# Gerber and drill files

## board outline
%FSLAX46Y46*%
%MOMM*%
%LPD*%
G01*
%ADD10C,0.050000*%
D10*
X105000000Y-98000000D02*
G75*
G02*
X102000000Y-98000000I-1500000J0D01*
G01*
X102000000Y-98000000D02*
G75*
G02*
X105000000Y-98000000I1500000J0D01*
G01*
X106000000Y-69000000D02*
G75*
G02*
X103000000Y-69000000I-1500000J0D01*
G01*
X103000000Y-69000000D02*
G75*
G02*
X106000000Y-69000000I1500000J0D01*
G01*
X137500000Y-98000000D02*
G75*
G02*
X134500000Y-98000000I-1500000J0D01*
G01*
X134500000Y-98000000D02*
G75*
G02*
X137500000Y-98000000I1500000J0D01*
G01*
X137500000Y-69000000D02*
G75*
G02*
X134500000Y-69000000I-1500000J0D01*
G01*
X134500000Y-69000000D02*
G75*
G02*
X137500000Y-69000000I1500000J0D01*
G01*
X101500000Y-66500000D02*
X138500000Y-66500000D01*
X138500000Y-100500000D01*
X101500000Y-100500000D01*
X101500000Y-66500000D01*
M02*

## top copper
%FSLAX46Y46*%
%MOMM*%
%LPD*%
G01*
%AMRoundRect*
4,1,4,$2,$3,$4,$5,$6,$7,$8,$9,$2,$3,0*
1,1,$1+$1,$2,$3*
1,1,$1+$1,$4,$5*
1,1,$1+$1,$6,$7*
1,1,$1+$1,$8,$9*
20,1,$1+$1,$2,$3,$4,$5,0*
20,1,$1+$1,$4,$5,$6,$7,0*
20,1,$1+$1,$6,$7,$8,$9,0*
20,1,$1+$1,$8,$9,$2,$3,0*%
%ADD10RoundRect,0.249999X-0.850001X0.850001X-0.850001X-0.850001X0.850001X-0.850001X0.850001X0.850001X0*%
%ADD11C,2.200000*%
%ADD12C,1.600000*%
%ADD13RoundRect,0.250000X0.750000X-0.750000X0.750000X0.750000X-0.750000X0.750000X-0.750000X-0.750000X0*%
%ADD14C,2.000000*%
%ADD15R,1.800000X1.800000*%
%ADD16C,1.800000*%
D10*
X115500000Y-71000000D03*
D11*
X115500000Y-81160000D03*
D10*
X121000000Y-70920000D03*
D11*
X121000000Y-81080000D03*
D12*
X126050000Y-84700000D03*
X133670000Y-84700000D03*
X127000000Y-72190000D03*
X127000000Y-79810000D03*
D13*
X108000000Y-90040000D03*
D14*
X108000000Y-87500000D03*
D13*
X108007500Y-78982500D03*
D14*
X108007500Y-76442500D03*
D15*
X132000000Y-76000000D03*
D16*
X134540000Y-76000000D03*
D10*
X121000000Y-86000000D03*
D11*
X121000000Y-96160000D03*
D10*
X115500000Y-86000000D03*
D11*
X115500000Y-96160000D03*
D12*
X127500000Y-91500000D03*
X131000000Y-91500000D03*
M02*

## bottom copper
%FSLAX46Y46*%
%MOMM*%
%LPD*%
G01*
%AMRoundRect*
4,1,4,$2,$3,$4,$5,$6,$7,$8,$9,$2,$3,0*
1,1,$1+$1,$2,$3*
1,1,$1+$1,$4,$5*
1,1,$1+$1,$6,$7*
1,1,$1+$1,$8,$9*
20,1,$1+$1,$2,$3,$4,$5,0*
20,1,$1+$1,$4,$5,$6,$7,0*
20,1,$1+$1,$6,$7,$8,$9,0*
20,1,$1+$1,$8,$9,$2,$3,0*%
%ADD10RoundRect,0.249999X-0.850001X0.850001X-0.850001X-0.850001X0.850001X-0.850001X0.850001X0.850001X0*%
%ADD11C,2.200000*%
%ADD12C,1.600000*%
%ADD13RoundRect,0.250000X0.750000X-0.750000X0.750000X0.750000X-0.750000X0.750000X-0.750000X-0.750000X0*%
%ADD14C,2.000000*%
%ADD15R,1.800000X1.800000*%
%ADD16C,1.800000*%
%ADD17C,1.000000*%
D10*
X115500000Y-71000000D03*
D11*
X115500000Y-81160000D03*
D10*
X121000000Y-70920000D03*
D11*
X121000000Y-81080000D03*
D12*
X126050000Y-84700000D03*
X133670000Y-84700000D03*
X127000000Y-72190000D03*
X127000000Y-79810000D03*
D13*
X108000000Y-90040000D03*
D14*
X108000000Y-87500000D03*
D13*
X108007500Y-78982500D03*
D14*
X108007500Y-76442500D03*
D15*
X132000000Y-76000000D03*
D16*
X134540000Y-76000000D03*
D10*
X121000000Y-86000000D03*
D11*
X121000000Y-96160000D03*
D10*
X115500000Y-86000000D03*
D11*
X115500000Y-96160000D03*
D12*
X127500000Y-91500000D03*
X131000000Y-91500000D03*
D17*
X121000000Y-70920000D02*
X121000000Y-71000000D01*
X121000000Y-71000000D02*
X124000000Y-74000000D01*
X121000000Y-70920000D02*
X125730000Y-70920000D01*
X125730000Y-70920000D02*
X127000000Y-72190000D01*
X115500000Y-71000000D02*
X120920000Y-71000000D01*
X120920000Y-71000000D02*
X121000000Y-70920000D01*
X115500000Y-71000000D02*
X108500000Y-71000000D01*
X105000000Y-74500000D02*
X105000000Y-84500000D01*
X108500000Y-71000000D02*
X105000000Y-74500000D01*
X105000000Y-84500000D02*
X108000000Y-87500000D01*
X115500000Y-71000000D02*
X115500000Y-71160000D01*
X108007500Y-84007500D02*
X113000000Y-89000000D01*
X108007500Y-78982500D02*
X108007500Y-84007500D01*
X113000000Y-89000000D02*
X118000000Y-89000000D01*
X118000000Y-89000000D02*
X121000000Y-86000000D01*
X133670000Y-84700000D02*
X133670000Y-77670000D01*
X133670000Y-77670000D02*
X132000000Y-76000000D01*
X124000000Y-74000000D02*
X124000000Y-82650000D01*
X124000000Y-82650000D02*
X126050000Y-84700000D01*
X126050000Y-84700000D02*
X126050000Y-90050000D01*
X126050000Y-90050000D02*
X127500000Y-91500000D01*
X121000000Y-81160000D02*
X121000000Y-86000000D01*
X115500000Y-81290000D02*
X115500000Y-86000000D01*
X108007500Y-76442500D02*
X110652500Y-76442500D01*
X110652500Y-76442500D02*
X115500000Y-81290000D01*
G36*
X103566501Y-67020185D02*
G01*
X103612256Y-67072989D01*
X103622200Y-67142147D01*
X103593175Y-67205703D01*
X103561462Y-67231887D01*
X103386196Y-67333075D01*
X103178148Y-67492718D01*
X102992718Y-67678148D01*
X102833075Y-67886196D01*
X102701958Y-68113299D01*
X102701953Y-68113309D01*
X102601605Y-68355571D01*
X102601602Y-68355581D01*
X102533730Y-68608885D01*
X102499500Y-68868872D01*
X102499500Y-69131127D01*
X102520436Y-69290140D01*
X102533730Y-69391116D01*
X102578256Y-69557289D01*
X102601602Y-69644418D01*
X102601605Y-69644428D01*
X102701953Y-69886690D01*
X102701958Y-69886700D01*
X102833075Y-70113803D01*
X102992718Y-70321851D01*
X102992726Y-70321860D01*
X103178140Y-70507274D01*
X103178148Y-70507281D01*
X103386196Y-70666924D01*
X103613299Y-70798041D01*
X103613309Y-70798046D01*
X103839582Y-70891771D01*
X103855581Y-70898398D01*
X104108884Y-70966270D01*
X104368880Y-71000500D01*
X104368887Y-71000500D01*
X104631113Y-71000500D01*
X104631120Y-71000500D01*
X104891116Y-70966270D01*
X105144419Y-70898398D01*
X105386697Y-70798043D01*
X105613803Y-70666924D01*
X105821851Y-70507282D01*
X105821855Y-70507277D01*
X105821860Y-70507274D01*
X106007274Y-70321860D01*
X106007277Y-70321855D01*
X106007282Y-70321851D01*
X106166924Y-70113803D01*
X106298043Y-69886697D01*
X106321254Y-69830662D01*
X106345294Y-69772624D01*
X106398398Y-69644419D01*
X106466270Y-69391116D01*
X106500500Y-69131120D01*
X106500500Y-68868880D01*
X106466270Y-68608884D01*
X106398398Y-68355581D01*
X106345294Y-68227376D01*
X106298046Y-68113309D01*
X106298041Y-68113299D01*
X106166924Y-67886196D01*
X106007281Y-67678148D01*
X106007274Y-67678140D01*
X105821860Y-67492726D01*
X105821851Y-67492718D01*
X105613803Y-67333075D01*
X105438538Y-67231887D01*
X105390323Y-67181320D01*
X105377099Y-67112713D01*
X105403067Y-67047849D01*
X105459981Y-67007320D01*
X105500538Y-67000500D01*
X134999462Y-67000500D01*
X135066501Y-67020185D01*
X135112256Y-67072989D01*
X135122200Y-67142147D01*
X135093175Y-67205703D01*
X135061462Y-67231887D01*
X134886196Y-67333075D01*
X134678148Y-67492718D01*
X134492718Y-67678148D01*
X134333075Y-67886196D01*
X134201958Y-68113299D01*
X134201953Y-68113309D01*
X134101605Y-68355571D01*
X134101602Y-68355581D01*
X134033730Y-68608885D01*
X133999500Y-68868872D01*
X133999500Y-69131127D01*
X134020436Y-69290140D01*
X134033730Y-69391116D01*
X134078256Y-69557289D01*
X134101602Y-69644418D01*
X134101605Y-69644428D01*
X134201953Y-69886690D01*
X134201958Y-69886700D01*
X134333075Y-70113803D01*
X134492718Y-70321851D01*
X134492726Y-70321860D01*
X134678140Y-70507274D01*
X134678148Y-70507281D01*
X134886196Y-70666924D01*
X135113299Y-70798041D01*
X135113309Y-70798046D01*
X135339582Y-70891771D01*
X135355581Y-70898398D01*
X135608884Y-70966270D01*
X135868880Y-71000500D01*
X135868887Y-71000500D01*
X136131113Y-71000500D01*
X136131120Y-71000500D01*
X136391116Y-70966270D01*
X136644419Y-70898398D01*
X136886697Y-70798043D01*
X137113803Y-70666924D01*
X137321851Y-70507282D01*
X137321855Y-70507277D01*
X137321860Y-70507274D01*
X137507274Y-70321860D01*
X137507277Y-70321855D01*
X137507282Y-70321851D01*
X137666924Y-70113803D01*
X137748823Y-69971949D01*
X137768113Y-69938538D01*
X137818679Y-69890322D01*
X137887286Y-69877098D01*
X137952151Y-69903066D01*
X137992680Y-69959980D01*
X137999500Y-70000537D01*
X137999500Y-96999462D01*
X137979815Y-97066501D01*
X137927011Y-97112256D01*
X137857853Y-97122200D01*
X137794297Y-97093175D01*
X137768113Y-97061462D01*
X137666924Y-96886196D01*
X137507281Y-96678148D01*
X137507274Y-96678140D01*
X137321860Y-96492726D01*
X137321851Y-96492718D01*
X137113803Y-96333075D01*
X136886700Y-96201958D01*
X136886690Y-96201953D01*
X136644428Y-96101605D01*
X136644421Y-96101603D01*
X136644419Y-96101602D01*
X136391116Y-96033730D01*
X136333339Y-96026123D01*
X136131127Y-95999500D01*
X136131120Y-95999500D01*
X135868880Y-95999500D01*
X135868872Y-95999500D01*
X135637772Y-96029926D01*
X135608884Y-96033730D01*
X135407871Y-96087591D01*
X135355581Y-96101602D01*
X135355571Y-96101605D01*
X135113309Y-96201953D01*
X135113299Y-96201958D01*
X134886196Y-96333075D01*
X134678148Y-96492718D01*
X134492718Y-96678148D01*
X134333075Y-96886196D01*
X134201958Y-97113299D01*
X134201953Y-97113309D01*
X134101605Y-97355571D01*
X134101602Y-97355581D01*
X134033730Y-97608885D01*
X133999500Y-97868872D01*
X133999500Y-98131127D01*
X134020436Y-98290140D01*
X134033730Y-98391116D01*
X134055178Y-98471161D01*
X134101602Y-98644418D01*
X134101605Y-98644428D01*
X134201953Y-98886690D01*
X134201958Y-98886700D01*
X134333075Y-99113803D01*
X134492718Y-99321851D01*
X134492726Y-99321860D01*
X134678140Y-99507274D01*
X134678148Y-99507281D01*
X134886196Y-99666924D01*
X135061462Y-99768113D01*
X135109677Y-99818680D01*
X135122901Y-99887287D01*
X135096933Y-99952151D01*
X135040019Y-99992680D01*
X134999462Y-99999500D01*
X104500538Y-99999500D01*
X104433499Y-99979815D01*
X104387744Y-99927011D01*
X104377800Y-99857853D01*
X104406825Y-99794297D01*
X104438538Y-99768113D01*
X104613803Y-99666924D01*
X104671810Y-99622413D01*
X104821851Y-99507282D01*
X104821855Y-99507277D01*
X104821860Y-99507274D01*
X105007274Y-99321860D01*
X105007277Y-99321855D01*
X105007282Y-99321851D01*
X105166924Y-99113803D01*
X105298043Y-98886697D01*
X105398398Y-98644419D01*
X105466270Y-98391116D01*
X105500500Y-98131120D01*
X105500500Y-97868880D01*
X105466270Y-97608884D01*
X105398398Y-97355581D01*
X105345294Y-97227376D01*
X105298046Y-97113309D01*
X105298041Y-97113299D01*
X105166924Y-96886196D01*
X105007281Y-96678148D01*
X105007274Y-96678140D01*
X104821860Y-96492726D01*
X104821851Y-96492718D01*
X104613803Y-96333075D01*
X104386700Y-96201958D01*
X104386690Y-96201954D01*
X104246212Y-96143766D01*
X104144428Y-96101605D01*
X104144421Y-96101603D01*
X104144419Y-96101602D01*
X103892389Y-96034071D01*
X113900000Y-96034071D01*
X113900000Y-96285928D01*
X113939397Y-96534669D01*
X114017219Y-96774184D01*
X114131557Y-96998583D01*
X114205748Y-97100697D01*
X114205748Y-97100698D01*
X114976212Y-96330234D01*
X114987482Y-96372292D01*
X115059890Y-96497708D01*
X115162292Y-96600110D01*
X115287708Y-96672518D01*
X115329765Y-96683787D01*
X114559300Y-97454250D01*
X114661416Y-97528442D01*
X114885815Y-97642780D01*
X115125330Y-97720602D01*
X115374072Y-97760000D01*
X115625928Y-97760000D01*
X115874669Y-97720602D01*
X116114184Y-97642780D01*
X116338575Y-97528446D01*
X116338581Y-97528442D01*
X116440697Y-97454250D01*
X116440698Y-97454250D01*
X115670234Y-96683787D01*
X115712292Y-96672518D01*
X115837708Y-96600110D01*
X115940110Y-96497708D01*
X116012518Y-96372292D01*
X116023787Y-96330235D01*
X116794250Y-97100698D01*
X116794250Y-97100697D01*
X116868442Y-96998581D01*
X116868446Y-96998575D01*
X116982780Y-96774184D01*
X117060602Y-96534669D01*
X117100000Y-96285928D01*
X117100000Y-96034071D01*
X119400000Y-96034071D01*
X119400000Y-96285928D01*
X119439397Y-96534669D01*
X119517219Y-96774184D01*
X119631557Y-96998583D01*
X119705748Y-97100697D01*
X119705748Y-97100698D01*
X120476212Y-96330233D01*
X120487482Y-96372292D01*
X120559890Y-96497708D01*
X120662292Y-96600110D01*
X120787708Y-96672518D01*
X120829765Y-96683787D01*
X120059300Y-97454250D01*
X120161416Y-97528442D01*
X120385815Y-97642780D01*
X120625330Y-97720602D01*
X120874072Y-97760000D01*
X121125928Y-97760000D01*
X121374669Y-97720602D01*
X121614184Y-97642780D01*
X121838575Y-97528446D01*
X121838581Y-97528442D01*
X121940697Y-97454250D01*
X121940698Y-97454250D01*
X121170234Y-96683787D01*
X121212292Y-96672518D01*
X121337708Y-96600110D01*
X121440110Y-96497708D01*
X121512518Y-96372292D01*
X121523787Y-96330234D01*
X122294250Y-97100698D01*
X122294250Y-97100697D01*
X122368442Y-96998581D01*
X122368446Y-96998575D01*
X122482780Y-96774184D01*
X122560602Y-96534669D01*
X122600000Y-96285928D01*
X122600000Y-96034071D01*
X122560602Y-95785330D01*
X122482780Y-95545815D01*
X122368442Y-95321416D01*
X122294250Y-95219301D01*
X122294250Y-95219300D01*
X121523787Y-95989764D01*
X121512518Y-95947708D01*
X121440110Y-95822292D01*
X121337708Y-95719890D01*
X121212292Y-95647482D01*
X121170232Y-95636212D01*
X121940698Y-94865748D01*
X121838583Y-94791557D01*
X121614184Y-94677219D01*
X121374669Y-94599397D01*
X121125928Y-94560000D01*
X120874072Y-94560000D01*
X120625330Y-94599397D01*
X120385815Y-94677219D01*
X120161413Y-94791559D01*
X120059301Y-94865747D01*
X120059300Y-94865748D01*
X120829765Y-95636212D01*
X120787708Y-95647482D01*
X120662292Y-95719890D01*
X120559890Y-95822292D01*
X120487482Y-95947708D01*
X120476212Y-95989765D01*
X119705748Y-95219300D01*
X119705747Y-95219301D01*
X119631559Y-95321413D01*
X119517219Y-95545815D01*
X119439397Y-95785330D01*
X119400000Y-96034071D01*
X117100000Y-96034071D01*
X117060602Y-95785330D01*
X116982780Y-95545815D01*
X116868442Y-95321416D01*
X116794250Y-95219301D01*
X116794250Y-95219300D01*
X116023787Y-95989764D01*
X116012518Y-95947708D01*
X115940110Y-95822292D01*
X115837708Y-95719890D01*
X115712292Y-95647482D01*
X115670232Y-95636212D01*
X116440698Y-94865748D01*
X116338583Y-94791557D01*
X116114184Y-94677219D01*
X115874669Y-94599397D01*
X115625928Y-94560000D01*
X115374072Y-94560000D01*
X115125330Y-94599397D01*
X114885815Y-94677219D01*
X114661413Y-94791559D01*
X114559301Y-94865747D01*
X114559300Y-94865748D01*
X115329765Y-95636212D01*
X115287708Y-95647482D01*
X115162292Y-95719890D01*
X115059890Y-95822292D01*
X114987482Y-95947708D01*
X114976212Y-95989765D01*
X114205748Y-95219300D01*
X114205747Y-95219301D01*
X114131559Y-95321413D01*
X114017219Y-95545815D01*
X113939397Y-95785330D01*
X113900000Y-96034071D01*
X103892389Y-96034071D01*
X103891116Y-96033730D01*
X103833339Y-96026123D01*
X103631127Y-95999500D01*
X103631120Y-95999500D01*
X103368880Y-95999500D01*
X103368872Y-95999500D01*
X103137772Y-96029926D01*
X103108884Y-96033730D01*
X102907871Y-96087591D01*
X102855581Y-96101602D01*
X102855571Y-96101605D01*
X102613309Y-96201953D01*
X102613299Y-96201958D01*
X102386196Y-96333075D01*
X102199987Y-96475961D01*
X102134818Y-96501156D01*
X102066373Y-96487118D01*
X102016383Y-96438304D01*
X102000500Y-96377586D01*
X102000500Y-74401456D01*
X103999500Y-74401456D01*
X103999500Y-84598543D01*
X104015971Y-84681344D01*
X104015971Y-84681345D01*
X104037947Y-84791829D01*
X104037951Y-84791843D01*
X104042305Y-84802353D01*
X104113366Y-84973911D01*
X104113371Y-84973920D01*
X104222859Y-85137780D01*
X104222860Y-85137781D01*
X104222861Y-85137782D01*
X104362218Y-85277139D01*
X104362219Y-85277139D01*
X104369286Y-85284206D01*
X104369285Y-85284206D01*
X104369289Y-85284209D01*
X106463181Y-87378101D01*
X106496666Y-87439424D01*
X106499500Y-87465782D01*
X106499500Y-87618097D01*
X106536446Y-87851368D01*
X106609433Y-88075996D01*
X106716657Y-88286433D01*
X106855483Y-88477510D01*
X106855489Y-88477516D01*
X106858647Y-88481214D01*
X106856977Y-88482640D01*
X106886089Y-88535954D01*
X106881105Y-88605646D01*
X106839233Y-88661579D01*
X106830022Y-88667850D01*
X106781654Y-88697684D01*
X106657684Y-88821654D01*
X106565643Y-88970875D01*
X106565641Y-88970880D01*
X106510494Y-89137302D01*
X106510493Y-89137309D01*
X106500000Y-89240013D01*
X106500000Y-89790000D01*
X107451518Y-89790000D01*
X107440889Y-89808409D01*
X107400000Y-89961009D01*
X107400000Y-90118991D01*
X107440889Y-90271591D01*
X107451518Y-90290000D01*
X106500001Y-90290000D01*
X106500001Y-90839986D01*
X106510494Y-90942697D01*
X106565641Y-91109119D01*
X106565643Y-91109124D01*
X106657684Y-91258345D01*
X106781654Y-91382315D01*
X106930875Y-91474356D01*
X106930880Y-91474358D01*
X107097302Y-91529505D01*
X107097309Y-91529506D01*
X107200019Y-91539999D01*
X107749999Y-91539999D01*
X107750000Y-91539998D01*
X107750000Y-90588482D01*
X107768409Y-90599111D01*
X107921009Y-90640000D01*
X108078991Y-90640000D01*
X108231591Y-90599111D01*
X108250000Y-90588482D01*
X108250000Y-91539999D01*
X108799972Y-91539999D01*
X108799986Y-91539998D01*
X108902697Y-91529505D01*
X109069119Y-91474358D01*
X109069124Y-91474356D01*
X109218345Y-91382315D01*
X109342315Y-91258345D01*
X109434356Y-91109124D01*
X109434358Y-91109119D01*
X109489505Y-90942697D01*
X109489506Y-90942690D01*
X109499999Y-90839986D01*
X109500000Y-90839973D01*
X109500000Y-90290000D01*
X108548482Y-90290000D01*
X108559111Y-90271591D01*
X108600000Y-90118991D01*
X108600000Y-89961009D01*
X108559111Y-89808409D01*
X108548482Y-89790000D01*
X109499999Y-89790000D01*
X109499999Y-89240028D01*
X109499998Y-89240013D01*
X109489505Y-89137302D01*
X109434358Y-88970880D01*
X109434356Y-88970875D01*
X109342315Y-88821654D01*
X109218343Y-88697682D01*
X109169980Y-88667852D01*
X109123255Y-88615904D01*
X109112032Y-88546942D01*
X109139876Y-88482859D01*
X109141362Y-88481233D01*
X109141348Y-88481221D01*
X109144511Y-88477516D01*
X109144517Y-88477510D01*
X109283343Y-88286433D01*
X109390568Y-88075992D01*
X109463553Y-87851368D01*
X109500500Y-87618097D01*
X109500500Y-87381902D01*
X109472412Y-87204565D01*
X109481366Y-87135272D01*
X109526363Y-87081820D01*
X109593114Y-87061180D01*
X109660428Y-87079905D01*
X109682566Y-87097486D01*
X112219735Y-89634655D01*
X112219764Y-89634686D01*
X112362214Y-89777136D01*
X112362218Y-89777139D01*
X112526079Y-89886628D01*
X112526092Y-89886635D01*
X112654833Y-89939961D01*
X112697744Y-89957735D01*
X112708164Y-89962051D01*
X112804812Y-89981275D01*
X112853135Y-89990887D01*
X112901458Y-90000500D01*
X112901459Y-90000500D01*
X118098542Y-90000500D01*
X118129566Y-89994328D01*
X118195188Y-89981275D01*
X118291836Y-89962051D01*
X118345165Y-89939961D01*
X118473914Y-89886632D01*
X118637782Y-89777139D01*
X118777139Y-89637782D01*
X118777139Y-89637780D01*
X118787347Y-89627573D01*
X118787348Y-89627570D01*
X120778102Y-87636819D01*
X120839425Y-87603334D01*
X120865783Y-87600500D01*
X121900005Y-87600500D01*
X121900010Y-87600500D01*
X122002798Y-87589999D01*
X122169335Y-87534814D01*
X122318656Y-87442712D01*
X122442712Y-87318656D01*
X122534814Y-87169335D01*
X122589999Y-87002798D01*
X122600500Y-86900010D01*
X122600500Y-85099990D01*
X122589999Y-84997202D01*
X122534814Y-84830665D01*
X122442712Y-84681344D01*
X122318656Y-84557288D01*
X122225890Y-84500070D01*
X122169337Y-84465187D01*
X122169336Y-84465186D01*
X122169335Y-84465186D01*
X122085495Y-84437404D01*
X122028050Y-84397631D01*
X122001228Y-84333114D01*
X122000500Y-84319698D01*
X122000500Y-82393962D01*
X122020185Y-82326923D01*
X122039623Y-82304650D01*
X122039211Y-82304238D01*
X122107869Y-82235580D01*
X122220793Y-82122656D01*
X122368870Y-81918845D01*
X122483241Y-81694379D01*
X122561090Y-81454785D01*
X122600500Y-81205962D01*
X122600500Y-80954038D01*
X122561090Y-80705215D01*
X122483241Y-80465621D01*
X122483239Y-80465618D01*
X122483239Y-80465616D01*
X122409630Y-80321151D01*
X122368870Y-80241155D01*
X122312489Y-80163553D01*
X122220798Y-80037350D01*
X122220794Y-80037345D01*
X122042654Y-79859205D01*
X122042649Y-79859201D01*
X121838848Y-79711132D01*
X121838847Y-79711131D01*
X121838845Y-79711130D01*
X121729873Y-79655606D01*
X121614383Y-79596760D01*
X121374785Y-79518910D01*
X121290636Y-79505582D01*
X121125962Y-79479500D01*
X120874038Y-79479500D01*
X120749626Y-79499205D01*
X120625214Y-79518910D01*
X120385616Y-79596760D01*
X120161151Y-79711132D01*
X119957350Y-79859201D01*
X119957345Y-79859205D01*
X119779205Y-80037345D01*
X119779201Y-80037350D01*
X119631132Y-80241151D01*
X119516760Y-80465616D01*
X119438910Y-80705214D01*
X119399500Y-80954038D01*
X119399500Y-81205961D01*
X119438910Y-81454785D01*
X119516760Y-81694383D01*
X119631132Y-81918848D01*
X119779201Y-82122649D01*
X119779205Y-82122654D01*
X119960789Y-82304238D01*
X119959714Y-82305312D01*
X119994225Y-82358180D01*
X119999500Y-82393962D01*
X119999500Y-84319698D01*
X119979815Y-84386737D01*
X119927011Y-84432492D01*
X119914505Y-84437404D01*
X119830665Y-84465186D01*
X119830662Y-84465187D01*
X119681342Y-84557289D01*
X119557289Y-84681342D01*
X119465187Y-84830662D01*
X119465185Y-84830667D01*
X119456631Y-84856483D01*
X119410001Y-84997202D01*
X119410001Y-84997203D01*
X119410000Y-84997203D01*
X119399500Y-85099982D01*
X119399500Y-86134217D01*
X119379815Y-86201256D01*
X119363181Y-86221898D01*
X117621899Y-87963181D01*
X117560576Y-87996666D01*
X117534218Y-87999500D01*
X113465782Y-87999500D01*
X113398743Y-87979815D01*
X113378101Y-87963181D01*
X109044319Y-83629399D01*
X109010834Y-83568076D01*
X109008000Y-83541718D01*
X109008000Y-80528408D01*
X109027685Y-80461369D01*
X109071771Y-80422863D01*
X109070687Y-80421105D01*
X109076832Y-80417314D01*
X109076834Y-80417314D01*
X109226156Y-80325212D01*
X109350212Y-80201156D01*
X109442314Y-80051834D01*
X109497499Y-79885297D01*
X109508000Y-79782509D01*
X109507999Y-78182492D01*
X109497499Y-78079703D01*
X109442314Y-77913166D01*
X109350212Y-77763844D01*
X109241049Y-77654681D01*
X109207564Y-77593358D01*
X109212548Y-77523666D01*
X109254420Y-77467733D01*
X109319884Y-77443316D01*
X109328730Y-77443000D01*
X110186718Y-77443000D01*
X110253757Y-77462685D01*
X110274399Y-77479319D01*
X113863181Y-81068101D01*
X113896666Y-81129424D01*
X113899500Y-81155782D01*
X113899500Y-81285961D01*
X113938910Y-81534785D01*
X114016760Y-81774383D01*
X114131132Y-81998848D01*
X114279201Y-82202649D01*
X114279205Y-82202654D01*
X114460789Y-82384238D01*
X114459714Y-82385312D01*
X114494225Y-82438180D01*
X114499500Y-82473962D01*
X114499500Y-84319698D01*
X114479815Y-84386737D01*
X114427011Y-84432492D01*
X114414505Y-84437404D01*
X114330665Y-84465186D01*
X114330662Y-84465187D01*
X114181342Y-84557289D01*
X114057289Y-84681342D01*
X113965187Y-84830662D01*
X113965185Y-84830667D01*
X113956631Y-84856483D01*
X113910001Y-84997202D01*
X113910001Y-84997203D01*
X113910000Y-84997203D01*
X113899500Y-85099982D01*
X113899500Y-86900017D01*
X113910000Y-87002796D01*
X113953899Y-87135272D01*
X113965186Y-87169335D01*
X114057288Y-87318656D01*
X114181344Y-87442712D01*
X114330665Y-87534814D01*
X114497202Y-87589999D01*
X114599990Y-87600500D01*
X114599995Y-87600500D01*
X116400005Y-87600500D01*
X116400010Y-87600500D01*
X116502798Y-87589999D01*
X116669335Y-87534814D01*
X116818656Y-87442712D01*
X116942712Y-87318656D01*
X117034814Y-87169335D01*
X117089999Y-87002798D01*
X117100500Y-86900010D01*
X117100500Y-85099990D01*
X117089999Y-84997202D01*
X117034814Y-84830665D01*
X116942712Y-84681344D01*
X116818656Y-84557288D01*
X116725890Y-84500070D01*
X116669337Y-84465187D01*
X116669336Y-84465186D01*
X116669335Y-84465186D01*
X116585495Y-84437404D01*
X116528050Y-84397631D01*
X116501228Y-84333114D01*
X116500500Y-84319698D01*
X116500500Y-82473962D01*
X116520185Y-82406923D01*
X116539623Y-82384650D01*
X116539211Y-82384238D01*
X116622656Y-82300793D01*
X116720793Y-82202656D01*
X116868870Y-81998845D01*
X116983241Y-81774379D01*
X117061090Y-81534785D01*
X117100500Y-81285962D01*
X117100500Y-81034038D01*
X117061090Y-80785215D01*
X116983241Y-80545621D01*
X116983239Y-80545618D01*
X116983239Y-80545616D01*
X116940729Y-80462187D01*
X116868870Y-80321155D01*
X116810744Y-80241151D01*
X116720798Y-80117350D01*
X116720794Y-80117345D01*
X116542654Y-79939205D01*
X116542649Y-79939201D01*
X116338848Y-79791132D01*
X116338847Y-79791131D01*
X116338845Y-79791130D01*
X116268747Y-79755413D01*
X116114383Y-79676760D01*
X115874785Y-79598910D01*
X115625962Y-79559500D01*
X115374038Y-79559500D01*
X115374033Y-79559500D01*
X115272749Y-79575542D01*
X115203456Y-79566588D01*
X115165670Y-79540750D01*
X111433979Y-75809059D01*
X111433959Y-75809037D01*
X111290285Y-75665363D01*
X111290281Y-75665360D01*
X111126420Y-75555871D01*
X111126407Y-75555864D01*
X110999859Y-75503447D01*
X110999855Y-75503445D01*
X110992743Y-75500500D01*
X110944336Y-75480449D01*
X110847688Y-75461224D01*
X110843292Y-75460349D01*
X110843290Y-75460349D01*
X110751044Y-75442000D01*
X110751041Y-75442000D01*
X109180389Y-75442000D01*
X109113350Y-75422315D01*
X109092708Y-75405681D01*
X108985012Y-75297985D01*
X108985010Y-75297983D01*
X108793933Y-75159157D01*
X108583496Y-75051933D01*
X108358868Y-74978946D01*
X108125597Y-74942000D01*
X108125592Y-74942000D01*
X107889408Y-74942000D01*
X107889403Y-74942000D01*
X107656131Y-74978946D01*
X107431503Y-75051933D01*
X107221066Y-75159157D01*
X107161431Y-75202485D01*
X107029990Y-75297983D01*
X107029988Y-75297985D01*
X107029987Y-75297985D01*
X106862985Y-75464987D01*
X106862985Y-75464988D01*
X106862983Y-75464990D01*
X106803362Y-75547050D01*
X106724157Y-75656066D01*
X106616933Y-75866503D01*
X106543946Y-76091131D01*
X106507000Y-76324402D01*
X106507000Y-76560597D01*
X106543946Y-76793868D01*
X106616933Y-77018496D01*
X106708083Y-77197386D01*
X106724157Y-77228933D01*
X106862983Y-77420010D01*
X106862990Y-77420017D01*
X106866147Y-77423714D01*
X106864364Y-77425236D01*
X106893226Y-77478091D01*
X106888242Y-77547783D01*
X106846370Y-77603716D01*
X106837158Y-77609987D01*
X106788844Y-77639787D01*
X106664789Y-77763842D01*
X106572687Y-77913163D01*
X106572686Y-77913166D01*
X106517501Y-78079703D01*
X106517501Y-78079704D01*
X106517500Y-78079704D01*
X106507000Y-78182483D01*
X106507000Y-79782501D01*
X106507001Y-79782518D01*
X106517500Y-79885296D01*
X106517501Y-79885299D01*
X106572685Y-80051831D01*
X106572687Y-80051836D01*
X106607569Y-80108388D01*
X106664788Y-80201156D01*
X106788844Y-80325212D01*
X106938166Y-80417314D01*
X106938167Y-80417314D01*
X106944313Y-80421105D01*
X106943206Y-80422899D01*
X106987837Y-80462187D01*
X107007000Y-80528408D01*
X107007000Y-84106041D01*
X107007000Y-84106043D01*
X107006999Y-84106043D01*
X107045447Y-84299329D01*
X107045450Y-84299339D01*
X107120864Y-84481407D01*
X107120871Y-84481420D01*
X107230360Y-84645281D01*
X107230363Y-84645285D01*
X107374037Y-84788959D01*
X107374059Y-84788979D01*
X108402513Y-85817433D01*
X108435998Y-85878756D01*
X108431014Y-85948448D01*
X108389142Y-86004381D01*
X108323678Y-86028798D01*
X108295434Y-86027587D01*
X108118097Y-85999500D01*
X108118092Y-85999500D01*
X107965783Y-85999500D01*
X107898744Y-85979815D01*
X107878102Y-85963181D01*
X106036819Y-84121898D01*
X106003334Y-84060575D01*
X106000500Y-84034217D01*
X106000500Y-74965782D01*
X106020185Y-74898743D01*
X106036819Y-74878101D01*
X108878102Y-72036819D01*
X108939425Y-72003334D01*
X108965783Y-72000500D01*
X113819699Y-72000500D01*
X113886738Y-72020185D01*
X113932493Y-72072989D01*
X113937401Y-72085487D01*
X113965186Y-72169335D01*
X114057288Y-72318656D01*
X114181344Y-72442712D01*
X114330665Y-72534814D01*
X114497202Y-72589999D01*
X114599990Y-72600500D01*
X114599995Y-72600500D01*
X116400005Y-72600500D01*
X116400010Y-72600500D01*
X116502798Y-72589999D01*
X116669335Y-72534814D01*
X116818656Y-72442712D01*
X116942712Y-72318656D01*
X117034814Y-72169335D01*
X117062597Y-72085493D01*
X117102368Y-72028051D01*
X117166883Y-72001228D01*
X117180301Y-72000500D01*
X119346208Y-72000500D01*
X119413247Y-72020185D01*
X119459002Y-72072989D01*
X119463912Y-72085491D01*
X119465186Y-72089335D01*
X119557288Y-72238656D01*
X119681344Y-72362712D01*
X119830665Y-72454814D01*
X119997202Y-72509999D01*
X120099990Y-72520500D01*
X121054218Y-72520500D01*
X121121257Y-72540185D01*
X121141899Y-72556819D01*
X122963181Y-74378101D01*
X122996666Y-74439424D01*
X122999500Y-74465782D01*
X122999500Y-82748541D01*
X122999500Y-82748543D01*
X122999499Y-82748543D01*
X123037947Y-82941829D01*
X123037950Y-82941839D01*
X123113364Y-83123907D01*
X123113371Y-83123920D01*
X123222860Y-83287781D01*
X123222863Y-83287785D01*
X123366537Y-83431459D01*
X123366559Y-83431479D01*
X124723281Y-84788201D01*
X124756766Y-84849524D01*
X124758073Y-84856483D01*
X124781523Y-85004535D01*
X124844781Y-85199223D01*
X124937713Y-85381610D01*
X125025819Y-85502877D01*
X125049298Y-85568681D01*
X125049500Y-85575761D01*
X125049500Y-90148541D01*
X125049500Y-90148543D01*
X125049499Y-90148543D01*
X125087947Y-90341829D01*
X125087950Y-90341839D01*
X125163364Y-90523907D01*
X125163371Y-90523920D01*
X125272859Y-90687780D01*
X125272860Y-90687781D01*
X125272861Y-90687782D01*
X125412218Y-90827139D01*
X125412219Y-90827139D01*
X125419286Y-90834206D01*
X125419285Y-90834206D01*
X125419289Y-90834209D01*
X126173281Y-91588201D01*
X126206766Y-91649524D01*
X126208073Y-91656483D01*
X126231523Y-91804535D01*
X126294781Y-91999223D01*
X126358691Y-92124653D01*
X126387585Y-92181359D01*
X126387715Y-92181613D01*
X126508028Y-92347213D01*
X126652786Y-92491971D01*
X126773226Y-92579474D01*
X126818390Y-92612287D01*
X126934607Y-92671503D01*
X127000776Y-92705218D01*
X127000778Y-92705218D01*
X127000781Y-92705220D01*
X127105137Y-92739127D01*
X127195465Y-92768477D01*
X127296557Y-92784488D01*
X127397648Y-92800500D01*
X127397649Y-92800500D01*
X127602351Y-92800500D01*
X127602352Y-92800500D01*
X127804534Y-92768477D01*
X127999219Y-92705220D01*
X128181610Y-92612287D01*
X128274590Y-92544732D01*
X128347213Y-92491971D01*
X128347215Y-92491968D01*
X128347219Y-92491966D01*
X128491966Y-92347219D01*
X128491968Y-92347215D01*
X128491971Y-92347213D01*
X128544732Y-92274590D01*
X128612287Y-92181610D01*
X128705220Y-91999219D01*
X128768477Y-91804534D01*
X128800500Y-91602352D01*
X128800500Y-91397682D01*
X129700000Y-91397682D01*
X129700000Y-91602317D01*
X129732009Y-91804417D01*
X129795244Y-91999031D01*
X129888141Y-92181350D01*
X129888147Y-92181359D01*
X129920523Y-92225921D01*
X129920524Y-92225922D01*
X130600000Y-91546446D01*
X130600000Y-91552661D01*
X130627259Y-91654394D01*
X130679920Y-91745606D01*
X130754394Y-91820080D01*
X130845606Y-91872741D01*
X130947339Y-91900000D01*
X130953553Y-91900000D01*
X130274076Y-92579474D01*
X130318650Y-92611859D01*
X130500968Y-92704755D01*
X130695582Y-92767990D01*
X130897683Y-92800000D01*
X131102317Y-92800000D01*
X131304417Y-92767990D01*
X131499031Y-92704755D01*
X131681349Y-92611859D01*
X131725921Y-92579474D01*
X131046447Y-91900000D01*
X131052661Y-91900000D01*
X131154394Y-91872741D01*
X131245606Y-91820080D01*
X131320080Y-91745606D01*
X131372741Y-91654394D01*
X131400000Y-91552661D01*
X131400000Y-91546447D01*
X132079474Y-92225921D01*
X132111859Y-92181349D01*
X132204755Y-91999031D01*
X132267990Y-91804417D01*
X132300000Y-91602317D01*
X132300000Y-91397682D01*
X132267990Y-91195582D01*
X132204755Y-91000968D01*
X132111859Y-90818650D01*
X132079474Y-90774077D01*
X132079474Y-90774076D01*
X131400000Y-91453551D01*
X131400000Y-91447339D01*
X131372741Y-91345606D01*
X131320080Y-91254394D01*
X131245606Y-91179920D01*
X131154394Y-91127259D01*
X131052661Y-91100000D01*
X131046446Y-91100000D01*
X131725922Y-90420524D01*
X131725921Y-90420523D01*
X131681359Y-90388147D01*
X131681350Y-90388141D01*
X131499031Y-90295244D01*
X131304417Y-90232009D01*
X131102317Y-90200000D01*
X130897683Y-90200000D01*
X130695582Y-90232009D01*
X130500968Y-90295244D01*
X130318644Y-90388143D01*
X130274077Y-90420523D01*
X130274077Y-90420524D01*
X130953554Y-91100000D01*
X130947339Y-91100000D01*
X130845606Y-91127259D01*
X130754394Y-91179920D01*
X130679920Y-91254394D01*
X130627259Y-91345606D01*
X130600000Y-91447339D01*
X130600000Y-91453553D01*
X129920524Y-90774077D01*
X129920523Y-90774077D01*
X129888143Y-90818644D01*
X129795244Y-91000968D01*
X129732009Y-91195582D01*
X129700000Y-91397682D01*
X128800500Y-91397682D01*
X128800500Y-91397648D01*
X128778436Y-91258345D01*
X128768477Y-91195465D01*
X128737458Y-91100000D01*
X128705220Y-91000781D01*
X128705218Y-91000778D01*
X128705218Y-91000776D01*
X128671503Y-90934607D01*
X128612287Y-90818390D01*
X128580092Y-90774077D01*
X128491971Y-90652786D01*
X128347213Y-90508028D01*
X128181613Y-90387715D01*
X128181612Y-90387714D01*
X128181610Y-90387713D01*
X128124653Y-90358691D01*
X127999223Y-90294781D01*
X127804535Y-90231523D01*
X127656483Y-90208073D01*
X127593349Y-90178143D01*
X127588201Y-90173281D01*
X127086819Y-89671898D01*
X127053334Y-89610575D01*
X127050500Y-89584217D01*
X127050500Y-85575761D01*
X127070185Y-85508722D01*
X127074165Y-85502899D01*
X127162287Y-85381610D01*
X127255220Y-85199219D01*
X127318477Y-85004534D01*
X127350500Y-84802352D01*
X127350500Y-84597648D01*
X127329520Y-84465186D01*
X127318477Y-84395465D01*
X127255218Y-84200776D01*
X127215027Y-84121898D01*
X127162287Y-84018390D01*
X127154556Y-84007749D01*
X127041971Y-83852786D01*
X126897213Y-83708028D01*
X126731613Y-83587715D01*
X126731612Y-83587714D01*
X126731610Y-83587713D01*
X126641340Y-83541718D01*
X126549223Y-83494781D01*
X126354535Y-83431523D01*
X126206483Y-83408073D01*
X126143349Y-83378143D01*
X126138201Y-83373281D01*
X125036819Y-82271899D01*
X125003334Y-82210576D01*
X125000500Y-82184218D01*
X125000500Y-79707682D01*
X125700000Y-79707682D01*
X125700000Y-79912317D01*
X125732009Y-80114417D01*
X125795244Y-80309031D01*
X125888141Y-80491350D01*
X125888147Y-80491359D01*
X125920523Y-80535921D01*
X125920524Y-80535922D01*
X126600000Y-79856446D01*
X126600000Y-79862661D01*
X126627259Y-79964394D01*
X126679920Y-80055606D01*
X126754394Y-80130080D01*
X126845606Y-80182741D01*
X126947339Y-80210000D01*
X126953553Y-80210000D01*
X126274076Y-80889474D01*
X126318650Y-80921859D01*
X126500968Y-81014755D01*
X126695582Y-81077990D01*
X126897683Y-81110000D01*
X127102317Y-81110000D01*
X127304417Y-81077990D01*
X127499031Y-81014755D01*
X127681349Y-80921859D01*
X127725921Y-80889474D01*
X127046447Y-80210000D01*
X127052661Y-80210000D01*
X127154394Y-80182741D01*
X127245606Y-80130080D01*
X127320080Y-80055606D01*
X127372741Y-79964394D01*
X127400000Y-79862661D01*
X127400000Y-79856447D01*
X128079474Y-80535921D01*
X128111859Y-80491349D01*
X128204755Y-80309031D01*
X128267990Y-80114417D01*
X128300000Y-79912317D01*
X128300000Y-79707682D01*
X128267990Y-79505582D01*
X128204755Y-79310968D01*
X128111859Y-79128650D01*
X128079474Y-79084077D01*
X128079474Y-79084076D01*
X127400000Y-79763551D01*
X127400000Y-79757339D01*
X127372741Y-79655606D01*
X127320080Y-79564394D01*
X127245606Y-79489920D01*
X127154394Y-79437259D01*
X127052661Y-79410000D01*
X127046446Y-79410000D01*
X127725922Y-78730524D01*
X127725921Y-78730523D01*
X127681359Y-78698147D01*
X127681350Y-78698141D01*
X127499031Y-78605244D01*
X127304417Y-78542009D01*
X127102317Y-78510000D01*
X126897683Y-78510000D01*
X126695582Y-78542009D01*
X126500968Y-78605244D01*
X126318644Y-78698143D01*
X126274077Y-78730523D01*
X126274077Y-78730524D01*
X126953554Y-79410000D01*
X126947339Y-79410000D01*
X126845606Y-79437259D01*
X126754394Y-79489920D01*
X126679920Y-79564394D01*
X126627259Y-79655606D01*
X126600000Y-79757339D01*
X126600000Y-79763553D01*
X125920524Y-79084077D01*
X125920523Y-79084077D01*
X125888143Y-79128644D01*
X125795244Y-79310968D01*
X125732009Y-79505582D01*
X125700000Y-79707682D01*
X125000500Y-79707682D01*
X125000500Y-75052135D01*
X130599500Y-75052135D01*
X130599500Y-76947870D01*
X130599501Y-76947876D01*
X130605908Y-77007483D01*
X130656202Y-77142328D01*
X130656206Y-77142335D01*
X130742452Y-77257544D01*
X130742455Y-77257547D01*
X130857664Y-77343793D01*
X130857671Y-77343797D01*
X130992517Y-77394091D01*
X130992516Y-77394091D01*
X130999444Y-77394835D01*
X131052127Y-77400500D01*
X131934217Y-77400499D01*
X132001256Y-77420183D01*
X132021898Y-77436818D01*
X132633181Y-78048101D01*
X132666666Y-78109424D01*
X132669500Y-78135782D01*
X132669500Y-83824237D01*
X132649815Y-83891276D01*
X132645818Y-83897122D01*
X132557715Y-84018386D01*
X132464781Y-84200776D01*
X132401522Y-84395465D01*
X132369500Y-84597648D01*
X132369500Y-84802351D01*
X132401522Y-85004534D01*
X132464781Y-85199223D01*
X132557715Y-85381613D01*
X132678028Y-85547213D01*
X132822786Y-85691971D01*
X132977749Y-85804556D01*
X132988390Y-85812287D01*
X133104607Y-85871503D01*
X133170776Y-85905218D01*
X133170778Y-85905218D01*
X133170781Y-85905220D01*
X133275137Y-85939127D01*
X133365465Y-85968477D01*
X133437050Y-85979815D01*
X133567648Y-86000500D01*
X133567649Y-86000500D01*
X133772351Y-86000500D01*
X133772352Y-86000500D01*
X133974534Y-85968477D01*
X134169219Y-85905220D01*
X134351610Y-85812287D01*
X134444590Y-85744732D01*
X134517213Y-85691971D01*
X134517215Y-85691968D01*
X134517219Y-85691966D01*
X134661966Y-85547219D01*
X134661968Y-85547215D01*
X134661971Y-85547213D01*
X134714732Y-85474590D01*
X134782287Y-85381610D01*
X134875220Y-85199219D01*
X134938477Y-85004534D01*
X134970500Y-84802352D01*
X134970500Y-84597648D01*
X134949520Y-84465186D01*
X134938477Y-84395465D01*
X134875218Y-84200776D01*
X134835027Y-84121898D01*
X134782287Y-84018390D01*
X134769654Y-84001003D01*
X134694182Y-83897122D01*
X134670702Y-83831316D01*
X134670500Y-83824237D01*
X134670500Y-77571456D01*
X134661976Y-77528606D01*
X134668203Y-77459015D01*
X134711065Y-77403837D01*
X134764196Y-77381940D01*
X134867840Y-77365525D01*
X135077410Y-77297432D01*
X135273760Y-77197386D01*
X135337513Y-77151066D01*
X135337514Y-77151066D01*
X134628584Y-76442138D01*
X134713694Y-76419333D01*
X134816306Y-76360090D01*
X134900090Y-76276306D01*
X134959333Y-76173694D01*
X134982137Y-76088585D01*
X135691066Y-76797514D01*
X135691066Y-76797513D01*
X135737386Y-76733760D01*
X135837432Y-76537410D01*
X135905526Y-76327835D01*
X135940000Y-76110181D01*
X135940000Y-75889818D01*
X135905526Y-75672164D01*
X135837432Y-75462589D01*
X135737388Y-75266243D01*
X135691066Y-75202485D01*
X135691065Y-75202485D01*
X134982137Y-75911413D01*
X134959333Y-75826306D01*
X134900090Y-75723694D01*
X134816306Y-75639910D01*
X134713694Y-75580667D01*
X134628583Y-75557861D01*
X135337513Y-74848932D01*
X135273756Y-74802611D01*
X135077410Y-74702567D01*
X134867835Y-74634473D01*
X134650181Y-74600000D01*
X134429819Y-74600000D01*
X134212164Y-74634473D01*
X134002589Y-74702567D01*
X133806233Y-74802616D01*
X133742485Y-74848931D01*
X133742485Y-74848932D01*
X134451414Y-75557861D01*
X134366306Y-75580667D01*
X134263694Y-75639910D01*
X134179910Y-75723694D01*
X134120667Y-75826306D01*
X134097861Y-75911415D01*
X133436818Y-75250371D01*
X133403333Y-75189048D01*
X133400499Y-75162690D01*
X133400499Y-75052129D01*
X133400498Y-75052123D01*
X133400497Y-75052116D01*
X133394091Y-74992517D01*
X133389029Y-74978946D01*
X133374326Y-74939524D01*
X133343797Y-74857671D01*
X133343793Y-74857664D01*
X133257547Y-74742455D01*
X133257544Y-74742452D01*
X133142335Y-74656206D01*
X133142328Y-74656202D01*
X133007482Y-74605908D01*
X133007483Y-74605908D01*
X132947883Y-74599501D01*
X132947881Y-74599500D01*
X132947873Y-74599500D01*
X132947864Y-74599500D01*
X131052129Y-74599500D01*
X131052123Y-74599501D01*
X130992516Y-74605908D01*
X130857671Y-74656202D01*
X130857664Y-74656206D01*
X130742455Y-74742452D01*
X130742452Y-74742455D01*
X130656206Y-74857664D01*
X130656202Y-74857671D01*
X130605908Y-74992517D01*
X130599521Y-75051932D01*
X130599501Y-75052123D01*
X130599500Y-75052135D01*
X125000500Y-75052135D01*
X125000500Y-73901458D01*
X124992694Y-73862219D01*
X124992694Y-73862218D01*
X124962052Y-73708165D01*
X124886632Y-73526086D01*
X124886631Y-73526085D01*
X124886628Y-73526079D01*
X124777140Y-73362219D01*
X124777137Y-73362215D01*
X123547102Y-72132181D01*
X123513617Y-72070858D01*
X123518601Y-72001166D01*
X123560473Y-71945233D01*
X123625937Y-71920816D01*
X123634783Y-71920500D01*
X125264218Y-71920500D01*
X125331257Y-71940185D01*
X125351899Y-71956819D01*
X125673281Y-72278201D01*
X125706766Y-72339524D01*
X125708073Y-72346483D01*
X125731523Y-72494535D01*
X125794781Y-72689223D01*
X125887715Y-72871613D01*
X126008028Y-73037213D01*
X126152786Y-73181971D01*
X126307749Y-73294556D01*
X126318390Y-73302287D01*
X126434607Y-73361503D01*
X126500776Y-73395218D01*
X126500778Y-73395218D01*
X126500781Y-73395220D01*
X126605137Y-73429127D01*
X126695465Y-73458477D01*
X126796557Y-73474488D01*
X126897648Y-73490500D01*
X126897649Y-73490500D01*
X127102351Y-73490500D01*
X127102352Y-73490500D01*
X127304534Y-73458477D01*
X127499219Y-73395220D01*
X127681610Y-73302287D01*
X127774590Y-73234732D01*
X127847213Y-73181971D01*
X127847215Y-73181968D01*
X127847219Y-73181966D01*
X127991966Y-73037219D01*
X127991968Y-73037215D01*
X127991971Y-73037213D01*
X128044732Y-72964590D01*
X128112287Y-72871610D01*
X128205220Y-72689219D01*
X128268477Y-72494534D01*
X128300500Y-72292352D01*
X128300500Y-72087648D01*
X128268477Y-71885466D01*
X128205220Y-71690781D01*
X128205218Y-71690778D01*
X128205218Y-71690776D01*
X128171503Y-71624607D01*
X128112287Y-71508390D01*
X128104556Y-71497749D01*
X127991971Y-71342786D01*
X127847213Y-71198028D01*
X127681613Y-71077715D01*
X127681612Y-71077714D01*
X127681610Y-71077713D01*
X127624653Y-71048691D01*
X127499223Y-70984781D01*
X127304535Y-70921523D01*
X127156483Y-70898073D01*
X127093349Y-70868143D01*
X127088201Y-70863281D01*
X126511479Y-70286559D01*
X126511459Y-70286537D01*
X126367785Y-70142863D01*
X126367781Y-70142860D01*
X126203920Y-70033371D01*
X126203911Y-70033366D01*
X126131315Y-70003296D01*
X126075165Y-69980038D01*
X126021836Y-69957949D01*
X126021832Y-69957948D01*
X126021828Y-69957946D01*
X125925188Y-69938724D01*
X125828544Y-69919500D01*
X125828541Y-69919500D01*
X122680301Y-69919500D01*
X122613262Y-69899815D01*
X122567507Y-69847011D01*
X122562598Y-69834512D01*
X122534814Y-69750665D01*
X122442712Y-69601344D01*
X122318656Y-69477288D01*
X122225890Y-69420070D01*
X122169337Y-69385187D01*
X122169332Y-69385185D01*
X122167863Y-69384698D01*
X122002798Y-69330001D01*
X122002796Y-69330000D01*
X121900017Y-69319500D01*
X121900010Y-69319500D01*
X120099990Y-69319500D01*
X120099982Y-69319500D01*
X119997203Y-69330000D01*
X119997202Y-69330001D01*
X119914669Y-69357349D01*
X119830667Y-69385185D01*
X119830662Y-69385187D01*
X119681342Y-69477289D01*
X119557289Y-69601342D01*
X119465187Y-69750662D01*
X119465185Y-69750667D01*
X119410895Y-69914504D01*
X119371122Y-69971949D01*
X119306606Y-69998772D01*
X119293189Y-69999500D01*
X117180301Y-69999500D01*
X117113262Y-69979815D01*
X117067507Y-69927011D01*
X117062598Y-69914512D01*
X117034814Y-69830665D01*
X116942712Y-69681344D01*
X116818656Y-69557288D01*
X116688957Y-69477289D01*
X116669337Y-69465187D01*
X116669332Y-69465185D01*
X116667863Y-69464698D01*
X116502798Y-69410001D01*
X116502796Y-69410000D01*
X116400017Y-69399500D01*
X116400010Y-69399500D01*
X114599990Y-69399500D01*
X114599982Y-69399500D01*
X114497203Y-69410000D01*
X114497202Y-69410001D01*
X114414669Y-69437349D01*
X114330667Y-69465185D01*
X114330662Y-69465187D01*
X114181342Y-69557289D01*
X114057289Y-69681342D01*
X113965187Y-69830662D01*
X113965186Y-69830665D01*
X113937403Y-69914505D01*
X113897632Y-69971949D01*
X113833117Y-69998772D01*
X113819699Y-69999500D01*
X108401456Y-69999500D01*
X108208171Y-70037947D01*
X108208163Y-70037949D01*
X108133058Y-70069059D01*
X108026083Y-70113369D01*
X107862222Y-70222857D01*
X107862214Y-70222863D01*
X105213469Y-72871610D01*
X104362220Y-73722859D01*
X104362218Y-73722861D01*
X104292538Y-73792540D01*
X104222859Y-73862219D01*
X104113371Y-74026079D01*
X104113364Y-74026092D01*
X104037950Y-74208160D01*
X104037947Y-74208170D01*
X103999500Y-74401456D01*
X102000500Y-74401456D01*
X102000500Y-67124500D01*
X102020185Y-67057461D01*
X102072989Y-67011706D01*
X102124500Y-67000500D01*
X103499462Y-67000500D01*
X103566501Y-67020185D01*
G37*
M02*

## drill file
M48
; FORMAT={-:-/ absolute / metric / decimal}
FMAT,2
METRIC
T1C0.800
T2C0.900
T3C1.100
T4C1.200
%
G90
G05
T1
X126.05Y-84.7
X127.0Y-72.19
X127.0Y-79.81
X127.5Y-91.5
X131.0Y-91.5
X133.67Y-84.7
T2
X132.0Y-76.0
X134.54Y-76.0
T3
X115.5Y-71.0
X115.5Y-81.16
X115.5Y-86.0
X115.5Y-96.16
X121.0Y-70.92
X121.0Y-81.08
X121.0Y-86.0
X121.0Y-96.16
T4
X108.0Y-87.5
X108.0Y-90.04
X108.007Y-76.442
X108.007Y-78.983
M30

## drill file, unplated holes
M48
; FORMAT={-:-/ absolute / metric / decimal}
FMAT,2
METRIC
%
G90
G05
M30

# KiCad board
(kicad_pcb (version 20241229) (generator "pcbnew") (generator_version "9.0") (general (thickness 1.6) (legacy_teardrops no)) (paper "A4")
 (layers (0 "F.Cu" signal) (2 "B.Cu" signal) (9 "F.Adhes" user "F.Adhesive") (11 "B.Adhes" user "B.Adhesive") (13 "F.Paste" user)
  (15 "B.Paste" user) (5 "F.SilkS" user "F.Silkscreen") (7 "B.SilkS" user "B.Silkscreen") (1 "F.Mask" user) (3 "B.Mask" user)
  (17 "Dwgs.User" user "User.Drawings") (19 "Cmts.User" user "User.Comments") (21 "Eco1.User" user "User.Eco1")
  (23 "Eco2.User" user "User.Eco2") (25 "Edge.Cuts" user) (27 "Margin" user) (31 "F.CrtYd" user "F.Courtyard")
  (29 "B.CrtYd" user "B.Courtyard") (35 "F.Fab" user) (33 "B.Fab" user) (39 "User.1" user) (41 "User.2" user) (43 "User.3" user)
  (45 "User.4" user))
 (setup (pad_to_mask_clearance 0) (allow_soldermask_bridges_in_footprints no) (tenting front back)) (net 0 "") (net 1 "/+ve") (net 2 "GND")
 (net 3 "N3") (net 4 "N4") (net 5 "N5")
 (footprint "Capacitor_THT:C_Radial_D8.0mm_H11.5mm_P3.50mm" (layer "F.Cu") (at 127.5 91.5)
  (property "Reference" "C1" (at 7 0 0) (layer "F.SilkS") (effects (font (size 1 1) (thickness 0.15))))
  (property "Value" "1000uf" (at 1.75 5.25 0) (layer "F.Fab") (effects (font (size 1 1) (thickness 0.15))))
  (pad "1" thru_hole circle (at 0 0) (size 1.6 1.6) (drill 0.8) (layers "*.Cu" "*.Mask") (remove_unused_layers no) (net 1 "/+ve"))
  (pad "2" thru_hole circle (at 3.5 0) (size 1.6 1.6) (drill 0.8) (layers "*.Cu" "*.Mask") (remove_unused_layers no) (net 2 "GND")))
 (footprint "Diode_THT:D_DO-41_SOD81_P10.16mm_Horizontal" (layer "F.Cu") (at 121 86 -90)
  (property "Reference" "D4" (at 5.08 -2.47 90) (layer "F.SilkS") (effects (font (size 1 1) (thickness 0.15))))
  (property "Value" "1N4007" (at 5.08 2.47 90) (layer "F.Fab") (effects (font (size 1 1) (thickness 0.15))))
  (pad "1" thru_hole roundrect (at 0 0 270) (size 2.2 2.2) (drill 1.1) (layers "*.Cu" "*.Mask") (remove_unused_layers no)
   (roundrect_rratio 0.113636) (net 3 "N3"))
  (pad "2" thru_hole circle (at 10.16 0 270) (size 2.2 2.2) (drill 1.1) (layers "*.Cu" "*.Mask") (remove_unused_layers no) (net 2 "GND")))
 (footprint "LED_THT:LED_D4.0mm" (layer "F.Cu") (at 132 76)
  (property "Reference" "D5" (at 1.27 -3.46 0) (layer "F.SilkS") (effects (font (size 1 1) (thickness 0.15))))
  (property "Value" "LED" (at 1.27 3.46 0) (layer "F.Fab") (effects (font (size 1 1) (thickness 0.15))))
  (pad "1" thru_hole rect (at 0 0) (size 1.8 1.8) (drill 0.9) (layers "*.Cu" "*.Mask") (remove_unused_layers no) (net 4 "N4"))
  (pad "2" thru_hole circle (at 2.54 0) (size 1.8 1.8) (drill 0.9) (layers "*.Cu" "*.Mask") (remove_unused_layers no) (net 2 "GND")))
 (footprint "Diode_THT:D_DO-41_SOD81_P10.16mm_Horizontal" (layer "F.Cu") (at 115.5 71 -90)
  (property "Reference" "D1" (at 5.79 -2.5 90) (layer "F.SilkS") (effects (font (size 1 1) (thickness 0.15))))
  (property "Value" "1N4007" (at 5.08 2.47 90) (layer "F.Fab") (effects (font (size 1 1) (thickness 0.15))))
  (pad "1" thru_hole roundrect (at 0 0 270) (size 2.2 2.2) (drill 1.1) (layers "*.Cu" "*.Mask") (remove_unused_layers no)
   (roundrect_rratio 0.113636) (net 1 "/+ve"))
  (pad "2" thru_hole circle (at 10.16 0 270) (size 2.2 2.2) (drill 1.1) (layers "*.Cu" "*.Mask") (remove_unused_layers no) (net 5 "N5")))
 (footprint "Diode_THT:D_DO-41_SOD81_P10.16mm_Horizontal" (layer "F.Cu") (at 121 70.92 -90)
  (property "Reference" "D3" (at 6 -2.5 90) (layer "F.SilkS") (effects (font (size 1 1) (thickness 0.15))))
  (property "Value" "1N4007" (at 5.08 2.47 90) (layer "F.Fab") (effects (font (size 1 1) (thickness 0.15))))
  (pad "1" thru_hole roundrect (at 0 0 270) (size 2.2 2.2) (drill 1.1) (layers "*.Cu" "*.Mask") (remove_unused_layers no)
   (roundrect_rratio 0.113636) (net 1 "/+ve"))
  (pad "2" thru_hole circle (at 10.16 0 270) (size 2.2 2.2) (drill 1.1) (layers "*.Cu" "*.Mask") (remove_unused_layers no) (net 3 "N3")))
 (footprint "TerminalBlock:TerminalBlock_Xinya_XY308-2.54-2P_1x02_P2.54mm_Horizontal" (layer "F.Cu") (at 108 90.04 90)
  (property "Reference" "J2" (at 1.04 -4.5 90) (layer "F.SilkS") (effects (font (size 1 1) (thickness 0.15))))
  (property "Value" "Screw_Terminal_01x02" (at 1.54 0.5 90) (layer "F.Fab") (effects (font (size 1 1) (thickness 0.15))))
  (pad "1" thru_hole roundrect (at 0 0 90) (size 2 2) (drill 1.2) (layers "*.Cu" "*.Mask") (remove_unused_layers no)
   (roundrect_rratio 0.125) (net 2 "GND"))
  (pad "2" thru_hole circle (at 2.54 0 90) (size 2 2) (drill 1.2) (layers "*.Cu" "*.Mask") (remove_unused_layers no) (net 1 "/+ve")))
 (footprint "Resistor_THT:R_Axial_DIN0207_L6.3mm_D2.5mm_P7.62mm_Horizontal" (layer "F.Cu") (at 127 72.19 -90)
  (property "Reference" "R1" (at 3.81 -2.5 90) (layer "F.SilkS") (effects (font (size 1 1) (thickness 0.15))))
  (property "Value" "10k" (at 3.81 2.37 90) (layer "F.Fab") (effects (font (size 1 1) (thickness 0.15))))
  (pad "1" thru_hole circle (at 0 0 270) (size 1.6 1.6) (drill 0.8) (layers "*.Cu" "*.Mask") (remove_unused_layers no) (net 1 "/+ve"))
  (pad "2" thru_hole circle (at 7.62 0 270) (size 1.6 1.6) (drill 0.8) (layers "*.Cu" "*.Mask") (remove_unused_layers no) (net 2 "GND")))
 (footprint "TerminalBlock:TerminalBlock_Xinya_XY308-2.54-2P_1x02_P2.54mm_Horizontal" (layer "F.Cu") (at 108.0075 78.9825 90)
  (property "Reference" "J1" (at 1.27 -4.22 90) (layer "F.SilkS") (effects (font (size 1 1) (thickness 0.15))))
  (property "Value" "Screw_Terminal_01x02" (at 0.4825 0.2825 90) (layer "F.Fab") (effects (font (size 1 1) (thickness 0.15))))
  (pad "1" thru_hole roundrect (at 0 0 90) (size 2 2) (drill 1.2) (layers "*.Cu" "*.Mask") (remove_unused_layers no)
   (roundrect_rratio 0.125) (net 3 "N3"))
  (pad "2" thru_hole circle (at 2.54 0 90) (size 2 2) (drill 1.2) (layers "*.Cu" "*.Mask") (remove_unused_layers no) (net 5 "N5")))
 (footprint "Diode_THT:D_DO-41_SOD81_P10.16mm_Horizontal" (layer "F.Cu") (at 115.5 86 -90)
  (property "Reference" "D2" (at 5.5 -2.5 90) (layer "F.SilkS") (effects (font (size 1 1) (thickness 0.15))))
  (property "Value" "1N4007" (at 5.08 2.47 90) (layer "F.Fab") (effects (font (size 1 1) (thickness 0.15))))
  (pad "1" thru_hole roundrect (at 0 0 270) (size 2.2 2.2) (drill 1.1) (layers "*.Cu" "*.Mask") (remove_unused_layers no)
   (roundrect_rratio 0.113636) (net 5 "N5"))
  (pad "2" thru_hole circle (at 10.16 0 270) (size 2.2 2.2) (drill 1.1) (layers "*.Cu" "*.Mask") (remove_unused_layers no) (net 2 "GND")))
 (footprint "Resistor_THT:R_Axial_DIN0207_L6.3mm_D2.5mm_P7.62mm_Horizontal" (layer "F.Cu") (at 126.05 84.7)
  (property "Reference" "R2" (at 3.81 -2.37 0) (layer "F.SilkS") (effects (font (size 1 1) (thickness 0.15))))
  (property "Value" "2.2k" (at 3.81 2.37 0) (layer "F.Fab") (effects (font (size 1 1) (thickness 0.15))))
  (pad "1" thru_hole circle (at 0 0) (size 1.6 1.6) (drill 0.8) (layers "*.Cu" "*.Mask") (remove_unused_layers no) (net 1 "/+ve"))
  (pad "2" thru_hole circle (at 7.62 0) (size 1.6 1.6) (drill 0.8) (layers "*.Cu" "*.Mask") (remove_unused_layers no) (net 4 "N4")))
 (gr_circle (center 103.5 98) (end 105 98) (stroke (width 0.05) (type default)) (fill no) (layer "Edge.Cuts"))
 (gr_circle (center 136 69) (end 137.5 69) (stroke (width 0.05) (type default)) (fill no) (layer "Edge.Cuts"))
 (gr_rect (start 101.5 66.5) (end 138.5 100.5) (stroke (width 0.05) (type default)) (fill no) (layer "Edge.Cuts"))
 (gr_circle (center 136 98) (end 137.5 98) (stroke (width 0.05) (type default)) (fill no) (layer "Edge.Cuts"))
 (gr_circle (center 104.5 69) (end 106 69) (stroke (width 0.05) (type default)) (fill no) (layer "Edge.Cuts"))
 (segment (start 105 74.5) (end 105 84.5) (width 1) (layer "B.Cu") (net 1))
 (segment (start 115.5 71) (end 120.92 71) (width 1) (layer "B.Cu") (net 1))
 (segment (start 120.92 71) (end 121 70.92) (width 1) (layer "B.Cu") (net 1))
 (segment (start 121 70.92) (end 125.73 70.92) (width 1) (layer "B.Cu") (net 1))
 (segment (start 126.05 90.05) (end 127.5 91.5) (width 1) (layer "B.Cu") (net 1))
 (segment (start 126.05 84.7) (end 126.05 90.05) (width 1) (layer "B.Cu") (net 1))
 (segment (start 121 70.92) (end 121 71) (width 1) (layer "B.Cu") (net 1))
 (segment (start 124 74) (end 124 82.65) (width 1) (layer "B.Cu") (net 1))
 (segment (start 124 82.65) (end 126.05 84.7) (width 1) (layer "B.Cu") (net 1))
 (segment (start 115.5 71) (end 108.5 71) (width 1) (layer "B.Cu") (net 1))
 (segment (start 108.5 71) (end 105 74.5) (width 1) (layer "B.Cu") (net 1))
 (segment (start 105 84.5) (end 108 87.5) (width 1) (layer "B.Cu") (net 1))
 (segment (start 125.73 70.92) (end 127 72.19) (width 1) (layer "B.Cu") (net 1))
 (segment (start 121 71) (end 124 74) (width 1) (layer "B.Cu") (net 1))
 (segment (start 115.5 71) (end 115.5 71.16) (width 1) (layer "B.Cu") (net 1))
 (segment (start 110.6525 76.4425) (end 115.5 81.29) (width 1) (layer "B.Cu") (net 5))
 (segment (start 108.0075 76.4425) (end 110.6525 76.4425) (width 1) (layer "B.Cu") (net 5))
 (segment (start 115.5 81.29) (end 115.5 86) (width 1) (layer "B.Cu") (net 5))
 (segment (start 118 89) (end 121 86) (width 1) (layer "B.Cu") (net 3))
 (segment (start 108.0075 84.0075) (end 113 89) (width 1) (layer "B.Cu") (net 3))
 (segment (start 108.0075 78.9825) (end 108.0075 84.0075) (width 1) (layer "B.Cu") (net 3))
 (segment (start 113 89) (end 118 89) (width 1) (layer "B.Cu") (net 3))
 (segment (start 121 81.16) (end 121 86) (width 1) (layer "B.Cu") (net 3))
 (segment (start 133.67 84.7) (end 133.67 77.67) (width 1) (layer "B.Cu") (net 4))
 (segment (start 133.67 77.67) (end 132 76) (width 1) (layer "B.Cu") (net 4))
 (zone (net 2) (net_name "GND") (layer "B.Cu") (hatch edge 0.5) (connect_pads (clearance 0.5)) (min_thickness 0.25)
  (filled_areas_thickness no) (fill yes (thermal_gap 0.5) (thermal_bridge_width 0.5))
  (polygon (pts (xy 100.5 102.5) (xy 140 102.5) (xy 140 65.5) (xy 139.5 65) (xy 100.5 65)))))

